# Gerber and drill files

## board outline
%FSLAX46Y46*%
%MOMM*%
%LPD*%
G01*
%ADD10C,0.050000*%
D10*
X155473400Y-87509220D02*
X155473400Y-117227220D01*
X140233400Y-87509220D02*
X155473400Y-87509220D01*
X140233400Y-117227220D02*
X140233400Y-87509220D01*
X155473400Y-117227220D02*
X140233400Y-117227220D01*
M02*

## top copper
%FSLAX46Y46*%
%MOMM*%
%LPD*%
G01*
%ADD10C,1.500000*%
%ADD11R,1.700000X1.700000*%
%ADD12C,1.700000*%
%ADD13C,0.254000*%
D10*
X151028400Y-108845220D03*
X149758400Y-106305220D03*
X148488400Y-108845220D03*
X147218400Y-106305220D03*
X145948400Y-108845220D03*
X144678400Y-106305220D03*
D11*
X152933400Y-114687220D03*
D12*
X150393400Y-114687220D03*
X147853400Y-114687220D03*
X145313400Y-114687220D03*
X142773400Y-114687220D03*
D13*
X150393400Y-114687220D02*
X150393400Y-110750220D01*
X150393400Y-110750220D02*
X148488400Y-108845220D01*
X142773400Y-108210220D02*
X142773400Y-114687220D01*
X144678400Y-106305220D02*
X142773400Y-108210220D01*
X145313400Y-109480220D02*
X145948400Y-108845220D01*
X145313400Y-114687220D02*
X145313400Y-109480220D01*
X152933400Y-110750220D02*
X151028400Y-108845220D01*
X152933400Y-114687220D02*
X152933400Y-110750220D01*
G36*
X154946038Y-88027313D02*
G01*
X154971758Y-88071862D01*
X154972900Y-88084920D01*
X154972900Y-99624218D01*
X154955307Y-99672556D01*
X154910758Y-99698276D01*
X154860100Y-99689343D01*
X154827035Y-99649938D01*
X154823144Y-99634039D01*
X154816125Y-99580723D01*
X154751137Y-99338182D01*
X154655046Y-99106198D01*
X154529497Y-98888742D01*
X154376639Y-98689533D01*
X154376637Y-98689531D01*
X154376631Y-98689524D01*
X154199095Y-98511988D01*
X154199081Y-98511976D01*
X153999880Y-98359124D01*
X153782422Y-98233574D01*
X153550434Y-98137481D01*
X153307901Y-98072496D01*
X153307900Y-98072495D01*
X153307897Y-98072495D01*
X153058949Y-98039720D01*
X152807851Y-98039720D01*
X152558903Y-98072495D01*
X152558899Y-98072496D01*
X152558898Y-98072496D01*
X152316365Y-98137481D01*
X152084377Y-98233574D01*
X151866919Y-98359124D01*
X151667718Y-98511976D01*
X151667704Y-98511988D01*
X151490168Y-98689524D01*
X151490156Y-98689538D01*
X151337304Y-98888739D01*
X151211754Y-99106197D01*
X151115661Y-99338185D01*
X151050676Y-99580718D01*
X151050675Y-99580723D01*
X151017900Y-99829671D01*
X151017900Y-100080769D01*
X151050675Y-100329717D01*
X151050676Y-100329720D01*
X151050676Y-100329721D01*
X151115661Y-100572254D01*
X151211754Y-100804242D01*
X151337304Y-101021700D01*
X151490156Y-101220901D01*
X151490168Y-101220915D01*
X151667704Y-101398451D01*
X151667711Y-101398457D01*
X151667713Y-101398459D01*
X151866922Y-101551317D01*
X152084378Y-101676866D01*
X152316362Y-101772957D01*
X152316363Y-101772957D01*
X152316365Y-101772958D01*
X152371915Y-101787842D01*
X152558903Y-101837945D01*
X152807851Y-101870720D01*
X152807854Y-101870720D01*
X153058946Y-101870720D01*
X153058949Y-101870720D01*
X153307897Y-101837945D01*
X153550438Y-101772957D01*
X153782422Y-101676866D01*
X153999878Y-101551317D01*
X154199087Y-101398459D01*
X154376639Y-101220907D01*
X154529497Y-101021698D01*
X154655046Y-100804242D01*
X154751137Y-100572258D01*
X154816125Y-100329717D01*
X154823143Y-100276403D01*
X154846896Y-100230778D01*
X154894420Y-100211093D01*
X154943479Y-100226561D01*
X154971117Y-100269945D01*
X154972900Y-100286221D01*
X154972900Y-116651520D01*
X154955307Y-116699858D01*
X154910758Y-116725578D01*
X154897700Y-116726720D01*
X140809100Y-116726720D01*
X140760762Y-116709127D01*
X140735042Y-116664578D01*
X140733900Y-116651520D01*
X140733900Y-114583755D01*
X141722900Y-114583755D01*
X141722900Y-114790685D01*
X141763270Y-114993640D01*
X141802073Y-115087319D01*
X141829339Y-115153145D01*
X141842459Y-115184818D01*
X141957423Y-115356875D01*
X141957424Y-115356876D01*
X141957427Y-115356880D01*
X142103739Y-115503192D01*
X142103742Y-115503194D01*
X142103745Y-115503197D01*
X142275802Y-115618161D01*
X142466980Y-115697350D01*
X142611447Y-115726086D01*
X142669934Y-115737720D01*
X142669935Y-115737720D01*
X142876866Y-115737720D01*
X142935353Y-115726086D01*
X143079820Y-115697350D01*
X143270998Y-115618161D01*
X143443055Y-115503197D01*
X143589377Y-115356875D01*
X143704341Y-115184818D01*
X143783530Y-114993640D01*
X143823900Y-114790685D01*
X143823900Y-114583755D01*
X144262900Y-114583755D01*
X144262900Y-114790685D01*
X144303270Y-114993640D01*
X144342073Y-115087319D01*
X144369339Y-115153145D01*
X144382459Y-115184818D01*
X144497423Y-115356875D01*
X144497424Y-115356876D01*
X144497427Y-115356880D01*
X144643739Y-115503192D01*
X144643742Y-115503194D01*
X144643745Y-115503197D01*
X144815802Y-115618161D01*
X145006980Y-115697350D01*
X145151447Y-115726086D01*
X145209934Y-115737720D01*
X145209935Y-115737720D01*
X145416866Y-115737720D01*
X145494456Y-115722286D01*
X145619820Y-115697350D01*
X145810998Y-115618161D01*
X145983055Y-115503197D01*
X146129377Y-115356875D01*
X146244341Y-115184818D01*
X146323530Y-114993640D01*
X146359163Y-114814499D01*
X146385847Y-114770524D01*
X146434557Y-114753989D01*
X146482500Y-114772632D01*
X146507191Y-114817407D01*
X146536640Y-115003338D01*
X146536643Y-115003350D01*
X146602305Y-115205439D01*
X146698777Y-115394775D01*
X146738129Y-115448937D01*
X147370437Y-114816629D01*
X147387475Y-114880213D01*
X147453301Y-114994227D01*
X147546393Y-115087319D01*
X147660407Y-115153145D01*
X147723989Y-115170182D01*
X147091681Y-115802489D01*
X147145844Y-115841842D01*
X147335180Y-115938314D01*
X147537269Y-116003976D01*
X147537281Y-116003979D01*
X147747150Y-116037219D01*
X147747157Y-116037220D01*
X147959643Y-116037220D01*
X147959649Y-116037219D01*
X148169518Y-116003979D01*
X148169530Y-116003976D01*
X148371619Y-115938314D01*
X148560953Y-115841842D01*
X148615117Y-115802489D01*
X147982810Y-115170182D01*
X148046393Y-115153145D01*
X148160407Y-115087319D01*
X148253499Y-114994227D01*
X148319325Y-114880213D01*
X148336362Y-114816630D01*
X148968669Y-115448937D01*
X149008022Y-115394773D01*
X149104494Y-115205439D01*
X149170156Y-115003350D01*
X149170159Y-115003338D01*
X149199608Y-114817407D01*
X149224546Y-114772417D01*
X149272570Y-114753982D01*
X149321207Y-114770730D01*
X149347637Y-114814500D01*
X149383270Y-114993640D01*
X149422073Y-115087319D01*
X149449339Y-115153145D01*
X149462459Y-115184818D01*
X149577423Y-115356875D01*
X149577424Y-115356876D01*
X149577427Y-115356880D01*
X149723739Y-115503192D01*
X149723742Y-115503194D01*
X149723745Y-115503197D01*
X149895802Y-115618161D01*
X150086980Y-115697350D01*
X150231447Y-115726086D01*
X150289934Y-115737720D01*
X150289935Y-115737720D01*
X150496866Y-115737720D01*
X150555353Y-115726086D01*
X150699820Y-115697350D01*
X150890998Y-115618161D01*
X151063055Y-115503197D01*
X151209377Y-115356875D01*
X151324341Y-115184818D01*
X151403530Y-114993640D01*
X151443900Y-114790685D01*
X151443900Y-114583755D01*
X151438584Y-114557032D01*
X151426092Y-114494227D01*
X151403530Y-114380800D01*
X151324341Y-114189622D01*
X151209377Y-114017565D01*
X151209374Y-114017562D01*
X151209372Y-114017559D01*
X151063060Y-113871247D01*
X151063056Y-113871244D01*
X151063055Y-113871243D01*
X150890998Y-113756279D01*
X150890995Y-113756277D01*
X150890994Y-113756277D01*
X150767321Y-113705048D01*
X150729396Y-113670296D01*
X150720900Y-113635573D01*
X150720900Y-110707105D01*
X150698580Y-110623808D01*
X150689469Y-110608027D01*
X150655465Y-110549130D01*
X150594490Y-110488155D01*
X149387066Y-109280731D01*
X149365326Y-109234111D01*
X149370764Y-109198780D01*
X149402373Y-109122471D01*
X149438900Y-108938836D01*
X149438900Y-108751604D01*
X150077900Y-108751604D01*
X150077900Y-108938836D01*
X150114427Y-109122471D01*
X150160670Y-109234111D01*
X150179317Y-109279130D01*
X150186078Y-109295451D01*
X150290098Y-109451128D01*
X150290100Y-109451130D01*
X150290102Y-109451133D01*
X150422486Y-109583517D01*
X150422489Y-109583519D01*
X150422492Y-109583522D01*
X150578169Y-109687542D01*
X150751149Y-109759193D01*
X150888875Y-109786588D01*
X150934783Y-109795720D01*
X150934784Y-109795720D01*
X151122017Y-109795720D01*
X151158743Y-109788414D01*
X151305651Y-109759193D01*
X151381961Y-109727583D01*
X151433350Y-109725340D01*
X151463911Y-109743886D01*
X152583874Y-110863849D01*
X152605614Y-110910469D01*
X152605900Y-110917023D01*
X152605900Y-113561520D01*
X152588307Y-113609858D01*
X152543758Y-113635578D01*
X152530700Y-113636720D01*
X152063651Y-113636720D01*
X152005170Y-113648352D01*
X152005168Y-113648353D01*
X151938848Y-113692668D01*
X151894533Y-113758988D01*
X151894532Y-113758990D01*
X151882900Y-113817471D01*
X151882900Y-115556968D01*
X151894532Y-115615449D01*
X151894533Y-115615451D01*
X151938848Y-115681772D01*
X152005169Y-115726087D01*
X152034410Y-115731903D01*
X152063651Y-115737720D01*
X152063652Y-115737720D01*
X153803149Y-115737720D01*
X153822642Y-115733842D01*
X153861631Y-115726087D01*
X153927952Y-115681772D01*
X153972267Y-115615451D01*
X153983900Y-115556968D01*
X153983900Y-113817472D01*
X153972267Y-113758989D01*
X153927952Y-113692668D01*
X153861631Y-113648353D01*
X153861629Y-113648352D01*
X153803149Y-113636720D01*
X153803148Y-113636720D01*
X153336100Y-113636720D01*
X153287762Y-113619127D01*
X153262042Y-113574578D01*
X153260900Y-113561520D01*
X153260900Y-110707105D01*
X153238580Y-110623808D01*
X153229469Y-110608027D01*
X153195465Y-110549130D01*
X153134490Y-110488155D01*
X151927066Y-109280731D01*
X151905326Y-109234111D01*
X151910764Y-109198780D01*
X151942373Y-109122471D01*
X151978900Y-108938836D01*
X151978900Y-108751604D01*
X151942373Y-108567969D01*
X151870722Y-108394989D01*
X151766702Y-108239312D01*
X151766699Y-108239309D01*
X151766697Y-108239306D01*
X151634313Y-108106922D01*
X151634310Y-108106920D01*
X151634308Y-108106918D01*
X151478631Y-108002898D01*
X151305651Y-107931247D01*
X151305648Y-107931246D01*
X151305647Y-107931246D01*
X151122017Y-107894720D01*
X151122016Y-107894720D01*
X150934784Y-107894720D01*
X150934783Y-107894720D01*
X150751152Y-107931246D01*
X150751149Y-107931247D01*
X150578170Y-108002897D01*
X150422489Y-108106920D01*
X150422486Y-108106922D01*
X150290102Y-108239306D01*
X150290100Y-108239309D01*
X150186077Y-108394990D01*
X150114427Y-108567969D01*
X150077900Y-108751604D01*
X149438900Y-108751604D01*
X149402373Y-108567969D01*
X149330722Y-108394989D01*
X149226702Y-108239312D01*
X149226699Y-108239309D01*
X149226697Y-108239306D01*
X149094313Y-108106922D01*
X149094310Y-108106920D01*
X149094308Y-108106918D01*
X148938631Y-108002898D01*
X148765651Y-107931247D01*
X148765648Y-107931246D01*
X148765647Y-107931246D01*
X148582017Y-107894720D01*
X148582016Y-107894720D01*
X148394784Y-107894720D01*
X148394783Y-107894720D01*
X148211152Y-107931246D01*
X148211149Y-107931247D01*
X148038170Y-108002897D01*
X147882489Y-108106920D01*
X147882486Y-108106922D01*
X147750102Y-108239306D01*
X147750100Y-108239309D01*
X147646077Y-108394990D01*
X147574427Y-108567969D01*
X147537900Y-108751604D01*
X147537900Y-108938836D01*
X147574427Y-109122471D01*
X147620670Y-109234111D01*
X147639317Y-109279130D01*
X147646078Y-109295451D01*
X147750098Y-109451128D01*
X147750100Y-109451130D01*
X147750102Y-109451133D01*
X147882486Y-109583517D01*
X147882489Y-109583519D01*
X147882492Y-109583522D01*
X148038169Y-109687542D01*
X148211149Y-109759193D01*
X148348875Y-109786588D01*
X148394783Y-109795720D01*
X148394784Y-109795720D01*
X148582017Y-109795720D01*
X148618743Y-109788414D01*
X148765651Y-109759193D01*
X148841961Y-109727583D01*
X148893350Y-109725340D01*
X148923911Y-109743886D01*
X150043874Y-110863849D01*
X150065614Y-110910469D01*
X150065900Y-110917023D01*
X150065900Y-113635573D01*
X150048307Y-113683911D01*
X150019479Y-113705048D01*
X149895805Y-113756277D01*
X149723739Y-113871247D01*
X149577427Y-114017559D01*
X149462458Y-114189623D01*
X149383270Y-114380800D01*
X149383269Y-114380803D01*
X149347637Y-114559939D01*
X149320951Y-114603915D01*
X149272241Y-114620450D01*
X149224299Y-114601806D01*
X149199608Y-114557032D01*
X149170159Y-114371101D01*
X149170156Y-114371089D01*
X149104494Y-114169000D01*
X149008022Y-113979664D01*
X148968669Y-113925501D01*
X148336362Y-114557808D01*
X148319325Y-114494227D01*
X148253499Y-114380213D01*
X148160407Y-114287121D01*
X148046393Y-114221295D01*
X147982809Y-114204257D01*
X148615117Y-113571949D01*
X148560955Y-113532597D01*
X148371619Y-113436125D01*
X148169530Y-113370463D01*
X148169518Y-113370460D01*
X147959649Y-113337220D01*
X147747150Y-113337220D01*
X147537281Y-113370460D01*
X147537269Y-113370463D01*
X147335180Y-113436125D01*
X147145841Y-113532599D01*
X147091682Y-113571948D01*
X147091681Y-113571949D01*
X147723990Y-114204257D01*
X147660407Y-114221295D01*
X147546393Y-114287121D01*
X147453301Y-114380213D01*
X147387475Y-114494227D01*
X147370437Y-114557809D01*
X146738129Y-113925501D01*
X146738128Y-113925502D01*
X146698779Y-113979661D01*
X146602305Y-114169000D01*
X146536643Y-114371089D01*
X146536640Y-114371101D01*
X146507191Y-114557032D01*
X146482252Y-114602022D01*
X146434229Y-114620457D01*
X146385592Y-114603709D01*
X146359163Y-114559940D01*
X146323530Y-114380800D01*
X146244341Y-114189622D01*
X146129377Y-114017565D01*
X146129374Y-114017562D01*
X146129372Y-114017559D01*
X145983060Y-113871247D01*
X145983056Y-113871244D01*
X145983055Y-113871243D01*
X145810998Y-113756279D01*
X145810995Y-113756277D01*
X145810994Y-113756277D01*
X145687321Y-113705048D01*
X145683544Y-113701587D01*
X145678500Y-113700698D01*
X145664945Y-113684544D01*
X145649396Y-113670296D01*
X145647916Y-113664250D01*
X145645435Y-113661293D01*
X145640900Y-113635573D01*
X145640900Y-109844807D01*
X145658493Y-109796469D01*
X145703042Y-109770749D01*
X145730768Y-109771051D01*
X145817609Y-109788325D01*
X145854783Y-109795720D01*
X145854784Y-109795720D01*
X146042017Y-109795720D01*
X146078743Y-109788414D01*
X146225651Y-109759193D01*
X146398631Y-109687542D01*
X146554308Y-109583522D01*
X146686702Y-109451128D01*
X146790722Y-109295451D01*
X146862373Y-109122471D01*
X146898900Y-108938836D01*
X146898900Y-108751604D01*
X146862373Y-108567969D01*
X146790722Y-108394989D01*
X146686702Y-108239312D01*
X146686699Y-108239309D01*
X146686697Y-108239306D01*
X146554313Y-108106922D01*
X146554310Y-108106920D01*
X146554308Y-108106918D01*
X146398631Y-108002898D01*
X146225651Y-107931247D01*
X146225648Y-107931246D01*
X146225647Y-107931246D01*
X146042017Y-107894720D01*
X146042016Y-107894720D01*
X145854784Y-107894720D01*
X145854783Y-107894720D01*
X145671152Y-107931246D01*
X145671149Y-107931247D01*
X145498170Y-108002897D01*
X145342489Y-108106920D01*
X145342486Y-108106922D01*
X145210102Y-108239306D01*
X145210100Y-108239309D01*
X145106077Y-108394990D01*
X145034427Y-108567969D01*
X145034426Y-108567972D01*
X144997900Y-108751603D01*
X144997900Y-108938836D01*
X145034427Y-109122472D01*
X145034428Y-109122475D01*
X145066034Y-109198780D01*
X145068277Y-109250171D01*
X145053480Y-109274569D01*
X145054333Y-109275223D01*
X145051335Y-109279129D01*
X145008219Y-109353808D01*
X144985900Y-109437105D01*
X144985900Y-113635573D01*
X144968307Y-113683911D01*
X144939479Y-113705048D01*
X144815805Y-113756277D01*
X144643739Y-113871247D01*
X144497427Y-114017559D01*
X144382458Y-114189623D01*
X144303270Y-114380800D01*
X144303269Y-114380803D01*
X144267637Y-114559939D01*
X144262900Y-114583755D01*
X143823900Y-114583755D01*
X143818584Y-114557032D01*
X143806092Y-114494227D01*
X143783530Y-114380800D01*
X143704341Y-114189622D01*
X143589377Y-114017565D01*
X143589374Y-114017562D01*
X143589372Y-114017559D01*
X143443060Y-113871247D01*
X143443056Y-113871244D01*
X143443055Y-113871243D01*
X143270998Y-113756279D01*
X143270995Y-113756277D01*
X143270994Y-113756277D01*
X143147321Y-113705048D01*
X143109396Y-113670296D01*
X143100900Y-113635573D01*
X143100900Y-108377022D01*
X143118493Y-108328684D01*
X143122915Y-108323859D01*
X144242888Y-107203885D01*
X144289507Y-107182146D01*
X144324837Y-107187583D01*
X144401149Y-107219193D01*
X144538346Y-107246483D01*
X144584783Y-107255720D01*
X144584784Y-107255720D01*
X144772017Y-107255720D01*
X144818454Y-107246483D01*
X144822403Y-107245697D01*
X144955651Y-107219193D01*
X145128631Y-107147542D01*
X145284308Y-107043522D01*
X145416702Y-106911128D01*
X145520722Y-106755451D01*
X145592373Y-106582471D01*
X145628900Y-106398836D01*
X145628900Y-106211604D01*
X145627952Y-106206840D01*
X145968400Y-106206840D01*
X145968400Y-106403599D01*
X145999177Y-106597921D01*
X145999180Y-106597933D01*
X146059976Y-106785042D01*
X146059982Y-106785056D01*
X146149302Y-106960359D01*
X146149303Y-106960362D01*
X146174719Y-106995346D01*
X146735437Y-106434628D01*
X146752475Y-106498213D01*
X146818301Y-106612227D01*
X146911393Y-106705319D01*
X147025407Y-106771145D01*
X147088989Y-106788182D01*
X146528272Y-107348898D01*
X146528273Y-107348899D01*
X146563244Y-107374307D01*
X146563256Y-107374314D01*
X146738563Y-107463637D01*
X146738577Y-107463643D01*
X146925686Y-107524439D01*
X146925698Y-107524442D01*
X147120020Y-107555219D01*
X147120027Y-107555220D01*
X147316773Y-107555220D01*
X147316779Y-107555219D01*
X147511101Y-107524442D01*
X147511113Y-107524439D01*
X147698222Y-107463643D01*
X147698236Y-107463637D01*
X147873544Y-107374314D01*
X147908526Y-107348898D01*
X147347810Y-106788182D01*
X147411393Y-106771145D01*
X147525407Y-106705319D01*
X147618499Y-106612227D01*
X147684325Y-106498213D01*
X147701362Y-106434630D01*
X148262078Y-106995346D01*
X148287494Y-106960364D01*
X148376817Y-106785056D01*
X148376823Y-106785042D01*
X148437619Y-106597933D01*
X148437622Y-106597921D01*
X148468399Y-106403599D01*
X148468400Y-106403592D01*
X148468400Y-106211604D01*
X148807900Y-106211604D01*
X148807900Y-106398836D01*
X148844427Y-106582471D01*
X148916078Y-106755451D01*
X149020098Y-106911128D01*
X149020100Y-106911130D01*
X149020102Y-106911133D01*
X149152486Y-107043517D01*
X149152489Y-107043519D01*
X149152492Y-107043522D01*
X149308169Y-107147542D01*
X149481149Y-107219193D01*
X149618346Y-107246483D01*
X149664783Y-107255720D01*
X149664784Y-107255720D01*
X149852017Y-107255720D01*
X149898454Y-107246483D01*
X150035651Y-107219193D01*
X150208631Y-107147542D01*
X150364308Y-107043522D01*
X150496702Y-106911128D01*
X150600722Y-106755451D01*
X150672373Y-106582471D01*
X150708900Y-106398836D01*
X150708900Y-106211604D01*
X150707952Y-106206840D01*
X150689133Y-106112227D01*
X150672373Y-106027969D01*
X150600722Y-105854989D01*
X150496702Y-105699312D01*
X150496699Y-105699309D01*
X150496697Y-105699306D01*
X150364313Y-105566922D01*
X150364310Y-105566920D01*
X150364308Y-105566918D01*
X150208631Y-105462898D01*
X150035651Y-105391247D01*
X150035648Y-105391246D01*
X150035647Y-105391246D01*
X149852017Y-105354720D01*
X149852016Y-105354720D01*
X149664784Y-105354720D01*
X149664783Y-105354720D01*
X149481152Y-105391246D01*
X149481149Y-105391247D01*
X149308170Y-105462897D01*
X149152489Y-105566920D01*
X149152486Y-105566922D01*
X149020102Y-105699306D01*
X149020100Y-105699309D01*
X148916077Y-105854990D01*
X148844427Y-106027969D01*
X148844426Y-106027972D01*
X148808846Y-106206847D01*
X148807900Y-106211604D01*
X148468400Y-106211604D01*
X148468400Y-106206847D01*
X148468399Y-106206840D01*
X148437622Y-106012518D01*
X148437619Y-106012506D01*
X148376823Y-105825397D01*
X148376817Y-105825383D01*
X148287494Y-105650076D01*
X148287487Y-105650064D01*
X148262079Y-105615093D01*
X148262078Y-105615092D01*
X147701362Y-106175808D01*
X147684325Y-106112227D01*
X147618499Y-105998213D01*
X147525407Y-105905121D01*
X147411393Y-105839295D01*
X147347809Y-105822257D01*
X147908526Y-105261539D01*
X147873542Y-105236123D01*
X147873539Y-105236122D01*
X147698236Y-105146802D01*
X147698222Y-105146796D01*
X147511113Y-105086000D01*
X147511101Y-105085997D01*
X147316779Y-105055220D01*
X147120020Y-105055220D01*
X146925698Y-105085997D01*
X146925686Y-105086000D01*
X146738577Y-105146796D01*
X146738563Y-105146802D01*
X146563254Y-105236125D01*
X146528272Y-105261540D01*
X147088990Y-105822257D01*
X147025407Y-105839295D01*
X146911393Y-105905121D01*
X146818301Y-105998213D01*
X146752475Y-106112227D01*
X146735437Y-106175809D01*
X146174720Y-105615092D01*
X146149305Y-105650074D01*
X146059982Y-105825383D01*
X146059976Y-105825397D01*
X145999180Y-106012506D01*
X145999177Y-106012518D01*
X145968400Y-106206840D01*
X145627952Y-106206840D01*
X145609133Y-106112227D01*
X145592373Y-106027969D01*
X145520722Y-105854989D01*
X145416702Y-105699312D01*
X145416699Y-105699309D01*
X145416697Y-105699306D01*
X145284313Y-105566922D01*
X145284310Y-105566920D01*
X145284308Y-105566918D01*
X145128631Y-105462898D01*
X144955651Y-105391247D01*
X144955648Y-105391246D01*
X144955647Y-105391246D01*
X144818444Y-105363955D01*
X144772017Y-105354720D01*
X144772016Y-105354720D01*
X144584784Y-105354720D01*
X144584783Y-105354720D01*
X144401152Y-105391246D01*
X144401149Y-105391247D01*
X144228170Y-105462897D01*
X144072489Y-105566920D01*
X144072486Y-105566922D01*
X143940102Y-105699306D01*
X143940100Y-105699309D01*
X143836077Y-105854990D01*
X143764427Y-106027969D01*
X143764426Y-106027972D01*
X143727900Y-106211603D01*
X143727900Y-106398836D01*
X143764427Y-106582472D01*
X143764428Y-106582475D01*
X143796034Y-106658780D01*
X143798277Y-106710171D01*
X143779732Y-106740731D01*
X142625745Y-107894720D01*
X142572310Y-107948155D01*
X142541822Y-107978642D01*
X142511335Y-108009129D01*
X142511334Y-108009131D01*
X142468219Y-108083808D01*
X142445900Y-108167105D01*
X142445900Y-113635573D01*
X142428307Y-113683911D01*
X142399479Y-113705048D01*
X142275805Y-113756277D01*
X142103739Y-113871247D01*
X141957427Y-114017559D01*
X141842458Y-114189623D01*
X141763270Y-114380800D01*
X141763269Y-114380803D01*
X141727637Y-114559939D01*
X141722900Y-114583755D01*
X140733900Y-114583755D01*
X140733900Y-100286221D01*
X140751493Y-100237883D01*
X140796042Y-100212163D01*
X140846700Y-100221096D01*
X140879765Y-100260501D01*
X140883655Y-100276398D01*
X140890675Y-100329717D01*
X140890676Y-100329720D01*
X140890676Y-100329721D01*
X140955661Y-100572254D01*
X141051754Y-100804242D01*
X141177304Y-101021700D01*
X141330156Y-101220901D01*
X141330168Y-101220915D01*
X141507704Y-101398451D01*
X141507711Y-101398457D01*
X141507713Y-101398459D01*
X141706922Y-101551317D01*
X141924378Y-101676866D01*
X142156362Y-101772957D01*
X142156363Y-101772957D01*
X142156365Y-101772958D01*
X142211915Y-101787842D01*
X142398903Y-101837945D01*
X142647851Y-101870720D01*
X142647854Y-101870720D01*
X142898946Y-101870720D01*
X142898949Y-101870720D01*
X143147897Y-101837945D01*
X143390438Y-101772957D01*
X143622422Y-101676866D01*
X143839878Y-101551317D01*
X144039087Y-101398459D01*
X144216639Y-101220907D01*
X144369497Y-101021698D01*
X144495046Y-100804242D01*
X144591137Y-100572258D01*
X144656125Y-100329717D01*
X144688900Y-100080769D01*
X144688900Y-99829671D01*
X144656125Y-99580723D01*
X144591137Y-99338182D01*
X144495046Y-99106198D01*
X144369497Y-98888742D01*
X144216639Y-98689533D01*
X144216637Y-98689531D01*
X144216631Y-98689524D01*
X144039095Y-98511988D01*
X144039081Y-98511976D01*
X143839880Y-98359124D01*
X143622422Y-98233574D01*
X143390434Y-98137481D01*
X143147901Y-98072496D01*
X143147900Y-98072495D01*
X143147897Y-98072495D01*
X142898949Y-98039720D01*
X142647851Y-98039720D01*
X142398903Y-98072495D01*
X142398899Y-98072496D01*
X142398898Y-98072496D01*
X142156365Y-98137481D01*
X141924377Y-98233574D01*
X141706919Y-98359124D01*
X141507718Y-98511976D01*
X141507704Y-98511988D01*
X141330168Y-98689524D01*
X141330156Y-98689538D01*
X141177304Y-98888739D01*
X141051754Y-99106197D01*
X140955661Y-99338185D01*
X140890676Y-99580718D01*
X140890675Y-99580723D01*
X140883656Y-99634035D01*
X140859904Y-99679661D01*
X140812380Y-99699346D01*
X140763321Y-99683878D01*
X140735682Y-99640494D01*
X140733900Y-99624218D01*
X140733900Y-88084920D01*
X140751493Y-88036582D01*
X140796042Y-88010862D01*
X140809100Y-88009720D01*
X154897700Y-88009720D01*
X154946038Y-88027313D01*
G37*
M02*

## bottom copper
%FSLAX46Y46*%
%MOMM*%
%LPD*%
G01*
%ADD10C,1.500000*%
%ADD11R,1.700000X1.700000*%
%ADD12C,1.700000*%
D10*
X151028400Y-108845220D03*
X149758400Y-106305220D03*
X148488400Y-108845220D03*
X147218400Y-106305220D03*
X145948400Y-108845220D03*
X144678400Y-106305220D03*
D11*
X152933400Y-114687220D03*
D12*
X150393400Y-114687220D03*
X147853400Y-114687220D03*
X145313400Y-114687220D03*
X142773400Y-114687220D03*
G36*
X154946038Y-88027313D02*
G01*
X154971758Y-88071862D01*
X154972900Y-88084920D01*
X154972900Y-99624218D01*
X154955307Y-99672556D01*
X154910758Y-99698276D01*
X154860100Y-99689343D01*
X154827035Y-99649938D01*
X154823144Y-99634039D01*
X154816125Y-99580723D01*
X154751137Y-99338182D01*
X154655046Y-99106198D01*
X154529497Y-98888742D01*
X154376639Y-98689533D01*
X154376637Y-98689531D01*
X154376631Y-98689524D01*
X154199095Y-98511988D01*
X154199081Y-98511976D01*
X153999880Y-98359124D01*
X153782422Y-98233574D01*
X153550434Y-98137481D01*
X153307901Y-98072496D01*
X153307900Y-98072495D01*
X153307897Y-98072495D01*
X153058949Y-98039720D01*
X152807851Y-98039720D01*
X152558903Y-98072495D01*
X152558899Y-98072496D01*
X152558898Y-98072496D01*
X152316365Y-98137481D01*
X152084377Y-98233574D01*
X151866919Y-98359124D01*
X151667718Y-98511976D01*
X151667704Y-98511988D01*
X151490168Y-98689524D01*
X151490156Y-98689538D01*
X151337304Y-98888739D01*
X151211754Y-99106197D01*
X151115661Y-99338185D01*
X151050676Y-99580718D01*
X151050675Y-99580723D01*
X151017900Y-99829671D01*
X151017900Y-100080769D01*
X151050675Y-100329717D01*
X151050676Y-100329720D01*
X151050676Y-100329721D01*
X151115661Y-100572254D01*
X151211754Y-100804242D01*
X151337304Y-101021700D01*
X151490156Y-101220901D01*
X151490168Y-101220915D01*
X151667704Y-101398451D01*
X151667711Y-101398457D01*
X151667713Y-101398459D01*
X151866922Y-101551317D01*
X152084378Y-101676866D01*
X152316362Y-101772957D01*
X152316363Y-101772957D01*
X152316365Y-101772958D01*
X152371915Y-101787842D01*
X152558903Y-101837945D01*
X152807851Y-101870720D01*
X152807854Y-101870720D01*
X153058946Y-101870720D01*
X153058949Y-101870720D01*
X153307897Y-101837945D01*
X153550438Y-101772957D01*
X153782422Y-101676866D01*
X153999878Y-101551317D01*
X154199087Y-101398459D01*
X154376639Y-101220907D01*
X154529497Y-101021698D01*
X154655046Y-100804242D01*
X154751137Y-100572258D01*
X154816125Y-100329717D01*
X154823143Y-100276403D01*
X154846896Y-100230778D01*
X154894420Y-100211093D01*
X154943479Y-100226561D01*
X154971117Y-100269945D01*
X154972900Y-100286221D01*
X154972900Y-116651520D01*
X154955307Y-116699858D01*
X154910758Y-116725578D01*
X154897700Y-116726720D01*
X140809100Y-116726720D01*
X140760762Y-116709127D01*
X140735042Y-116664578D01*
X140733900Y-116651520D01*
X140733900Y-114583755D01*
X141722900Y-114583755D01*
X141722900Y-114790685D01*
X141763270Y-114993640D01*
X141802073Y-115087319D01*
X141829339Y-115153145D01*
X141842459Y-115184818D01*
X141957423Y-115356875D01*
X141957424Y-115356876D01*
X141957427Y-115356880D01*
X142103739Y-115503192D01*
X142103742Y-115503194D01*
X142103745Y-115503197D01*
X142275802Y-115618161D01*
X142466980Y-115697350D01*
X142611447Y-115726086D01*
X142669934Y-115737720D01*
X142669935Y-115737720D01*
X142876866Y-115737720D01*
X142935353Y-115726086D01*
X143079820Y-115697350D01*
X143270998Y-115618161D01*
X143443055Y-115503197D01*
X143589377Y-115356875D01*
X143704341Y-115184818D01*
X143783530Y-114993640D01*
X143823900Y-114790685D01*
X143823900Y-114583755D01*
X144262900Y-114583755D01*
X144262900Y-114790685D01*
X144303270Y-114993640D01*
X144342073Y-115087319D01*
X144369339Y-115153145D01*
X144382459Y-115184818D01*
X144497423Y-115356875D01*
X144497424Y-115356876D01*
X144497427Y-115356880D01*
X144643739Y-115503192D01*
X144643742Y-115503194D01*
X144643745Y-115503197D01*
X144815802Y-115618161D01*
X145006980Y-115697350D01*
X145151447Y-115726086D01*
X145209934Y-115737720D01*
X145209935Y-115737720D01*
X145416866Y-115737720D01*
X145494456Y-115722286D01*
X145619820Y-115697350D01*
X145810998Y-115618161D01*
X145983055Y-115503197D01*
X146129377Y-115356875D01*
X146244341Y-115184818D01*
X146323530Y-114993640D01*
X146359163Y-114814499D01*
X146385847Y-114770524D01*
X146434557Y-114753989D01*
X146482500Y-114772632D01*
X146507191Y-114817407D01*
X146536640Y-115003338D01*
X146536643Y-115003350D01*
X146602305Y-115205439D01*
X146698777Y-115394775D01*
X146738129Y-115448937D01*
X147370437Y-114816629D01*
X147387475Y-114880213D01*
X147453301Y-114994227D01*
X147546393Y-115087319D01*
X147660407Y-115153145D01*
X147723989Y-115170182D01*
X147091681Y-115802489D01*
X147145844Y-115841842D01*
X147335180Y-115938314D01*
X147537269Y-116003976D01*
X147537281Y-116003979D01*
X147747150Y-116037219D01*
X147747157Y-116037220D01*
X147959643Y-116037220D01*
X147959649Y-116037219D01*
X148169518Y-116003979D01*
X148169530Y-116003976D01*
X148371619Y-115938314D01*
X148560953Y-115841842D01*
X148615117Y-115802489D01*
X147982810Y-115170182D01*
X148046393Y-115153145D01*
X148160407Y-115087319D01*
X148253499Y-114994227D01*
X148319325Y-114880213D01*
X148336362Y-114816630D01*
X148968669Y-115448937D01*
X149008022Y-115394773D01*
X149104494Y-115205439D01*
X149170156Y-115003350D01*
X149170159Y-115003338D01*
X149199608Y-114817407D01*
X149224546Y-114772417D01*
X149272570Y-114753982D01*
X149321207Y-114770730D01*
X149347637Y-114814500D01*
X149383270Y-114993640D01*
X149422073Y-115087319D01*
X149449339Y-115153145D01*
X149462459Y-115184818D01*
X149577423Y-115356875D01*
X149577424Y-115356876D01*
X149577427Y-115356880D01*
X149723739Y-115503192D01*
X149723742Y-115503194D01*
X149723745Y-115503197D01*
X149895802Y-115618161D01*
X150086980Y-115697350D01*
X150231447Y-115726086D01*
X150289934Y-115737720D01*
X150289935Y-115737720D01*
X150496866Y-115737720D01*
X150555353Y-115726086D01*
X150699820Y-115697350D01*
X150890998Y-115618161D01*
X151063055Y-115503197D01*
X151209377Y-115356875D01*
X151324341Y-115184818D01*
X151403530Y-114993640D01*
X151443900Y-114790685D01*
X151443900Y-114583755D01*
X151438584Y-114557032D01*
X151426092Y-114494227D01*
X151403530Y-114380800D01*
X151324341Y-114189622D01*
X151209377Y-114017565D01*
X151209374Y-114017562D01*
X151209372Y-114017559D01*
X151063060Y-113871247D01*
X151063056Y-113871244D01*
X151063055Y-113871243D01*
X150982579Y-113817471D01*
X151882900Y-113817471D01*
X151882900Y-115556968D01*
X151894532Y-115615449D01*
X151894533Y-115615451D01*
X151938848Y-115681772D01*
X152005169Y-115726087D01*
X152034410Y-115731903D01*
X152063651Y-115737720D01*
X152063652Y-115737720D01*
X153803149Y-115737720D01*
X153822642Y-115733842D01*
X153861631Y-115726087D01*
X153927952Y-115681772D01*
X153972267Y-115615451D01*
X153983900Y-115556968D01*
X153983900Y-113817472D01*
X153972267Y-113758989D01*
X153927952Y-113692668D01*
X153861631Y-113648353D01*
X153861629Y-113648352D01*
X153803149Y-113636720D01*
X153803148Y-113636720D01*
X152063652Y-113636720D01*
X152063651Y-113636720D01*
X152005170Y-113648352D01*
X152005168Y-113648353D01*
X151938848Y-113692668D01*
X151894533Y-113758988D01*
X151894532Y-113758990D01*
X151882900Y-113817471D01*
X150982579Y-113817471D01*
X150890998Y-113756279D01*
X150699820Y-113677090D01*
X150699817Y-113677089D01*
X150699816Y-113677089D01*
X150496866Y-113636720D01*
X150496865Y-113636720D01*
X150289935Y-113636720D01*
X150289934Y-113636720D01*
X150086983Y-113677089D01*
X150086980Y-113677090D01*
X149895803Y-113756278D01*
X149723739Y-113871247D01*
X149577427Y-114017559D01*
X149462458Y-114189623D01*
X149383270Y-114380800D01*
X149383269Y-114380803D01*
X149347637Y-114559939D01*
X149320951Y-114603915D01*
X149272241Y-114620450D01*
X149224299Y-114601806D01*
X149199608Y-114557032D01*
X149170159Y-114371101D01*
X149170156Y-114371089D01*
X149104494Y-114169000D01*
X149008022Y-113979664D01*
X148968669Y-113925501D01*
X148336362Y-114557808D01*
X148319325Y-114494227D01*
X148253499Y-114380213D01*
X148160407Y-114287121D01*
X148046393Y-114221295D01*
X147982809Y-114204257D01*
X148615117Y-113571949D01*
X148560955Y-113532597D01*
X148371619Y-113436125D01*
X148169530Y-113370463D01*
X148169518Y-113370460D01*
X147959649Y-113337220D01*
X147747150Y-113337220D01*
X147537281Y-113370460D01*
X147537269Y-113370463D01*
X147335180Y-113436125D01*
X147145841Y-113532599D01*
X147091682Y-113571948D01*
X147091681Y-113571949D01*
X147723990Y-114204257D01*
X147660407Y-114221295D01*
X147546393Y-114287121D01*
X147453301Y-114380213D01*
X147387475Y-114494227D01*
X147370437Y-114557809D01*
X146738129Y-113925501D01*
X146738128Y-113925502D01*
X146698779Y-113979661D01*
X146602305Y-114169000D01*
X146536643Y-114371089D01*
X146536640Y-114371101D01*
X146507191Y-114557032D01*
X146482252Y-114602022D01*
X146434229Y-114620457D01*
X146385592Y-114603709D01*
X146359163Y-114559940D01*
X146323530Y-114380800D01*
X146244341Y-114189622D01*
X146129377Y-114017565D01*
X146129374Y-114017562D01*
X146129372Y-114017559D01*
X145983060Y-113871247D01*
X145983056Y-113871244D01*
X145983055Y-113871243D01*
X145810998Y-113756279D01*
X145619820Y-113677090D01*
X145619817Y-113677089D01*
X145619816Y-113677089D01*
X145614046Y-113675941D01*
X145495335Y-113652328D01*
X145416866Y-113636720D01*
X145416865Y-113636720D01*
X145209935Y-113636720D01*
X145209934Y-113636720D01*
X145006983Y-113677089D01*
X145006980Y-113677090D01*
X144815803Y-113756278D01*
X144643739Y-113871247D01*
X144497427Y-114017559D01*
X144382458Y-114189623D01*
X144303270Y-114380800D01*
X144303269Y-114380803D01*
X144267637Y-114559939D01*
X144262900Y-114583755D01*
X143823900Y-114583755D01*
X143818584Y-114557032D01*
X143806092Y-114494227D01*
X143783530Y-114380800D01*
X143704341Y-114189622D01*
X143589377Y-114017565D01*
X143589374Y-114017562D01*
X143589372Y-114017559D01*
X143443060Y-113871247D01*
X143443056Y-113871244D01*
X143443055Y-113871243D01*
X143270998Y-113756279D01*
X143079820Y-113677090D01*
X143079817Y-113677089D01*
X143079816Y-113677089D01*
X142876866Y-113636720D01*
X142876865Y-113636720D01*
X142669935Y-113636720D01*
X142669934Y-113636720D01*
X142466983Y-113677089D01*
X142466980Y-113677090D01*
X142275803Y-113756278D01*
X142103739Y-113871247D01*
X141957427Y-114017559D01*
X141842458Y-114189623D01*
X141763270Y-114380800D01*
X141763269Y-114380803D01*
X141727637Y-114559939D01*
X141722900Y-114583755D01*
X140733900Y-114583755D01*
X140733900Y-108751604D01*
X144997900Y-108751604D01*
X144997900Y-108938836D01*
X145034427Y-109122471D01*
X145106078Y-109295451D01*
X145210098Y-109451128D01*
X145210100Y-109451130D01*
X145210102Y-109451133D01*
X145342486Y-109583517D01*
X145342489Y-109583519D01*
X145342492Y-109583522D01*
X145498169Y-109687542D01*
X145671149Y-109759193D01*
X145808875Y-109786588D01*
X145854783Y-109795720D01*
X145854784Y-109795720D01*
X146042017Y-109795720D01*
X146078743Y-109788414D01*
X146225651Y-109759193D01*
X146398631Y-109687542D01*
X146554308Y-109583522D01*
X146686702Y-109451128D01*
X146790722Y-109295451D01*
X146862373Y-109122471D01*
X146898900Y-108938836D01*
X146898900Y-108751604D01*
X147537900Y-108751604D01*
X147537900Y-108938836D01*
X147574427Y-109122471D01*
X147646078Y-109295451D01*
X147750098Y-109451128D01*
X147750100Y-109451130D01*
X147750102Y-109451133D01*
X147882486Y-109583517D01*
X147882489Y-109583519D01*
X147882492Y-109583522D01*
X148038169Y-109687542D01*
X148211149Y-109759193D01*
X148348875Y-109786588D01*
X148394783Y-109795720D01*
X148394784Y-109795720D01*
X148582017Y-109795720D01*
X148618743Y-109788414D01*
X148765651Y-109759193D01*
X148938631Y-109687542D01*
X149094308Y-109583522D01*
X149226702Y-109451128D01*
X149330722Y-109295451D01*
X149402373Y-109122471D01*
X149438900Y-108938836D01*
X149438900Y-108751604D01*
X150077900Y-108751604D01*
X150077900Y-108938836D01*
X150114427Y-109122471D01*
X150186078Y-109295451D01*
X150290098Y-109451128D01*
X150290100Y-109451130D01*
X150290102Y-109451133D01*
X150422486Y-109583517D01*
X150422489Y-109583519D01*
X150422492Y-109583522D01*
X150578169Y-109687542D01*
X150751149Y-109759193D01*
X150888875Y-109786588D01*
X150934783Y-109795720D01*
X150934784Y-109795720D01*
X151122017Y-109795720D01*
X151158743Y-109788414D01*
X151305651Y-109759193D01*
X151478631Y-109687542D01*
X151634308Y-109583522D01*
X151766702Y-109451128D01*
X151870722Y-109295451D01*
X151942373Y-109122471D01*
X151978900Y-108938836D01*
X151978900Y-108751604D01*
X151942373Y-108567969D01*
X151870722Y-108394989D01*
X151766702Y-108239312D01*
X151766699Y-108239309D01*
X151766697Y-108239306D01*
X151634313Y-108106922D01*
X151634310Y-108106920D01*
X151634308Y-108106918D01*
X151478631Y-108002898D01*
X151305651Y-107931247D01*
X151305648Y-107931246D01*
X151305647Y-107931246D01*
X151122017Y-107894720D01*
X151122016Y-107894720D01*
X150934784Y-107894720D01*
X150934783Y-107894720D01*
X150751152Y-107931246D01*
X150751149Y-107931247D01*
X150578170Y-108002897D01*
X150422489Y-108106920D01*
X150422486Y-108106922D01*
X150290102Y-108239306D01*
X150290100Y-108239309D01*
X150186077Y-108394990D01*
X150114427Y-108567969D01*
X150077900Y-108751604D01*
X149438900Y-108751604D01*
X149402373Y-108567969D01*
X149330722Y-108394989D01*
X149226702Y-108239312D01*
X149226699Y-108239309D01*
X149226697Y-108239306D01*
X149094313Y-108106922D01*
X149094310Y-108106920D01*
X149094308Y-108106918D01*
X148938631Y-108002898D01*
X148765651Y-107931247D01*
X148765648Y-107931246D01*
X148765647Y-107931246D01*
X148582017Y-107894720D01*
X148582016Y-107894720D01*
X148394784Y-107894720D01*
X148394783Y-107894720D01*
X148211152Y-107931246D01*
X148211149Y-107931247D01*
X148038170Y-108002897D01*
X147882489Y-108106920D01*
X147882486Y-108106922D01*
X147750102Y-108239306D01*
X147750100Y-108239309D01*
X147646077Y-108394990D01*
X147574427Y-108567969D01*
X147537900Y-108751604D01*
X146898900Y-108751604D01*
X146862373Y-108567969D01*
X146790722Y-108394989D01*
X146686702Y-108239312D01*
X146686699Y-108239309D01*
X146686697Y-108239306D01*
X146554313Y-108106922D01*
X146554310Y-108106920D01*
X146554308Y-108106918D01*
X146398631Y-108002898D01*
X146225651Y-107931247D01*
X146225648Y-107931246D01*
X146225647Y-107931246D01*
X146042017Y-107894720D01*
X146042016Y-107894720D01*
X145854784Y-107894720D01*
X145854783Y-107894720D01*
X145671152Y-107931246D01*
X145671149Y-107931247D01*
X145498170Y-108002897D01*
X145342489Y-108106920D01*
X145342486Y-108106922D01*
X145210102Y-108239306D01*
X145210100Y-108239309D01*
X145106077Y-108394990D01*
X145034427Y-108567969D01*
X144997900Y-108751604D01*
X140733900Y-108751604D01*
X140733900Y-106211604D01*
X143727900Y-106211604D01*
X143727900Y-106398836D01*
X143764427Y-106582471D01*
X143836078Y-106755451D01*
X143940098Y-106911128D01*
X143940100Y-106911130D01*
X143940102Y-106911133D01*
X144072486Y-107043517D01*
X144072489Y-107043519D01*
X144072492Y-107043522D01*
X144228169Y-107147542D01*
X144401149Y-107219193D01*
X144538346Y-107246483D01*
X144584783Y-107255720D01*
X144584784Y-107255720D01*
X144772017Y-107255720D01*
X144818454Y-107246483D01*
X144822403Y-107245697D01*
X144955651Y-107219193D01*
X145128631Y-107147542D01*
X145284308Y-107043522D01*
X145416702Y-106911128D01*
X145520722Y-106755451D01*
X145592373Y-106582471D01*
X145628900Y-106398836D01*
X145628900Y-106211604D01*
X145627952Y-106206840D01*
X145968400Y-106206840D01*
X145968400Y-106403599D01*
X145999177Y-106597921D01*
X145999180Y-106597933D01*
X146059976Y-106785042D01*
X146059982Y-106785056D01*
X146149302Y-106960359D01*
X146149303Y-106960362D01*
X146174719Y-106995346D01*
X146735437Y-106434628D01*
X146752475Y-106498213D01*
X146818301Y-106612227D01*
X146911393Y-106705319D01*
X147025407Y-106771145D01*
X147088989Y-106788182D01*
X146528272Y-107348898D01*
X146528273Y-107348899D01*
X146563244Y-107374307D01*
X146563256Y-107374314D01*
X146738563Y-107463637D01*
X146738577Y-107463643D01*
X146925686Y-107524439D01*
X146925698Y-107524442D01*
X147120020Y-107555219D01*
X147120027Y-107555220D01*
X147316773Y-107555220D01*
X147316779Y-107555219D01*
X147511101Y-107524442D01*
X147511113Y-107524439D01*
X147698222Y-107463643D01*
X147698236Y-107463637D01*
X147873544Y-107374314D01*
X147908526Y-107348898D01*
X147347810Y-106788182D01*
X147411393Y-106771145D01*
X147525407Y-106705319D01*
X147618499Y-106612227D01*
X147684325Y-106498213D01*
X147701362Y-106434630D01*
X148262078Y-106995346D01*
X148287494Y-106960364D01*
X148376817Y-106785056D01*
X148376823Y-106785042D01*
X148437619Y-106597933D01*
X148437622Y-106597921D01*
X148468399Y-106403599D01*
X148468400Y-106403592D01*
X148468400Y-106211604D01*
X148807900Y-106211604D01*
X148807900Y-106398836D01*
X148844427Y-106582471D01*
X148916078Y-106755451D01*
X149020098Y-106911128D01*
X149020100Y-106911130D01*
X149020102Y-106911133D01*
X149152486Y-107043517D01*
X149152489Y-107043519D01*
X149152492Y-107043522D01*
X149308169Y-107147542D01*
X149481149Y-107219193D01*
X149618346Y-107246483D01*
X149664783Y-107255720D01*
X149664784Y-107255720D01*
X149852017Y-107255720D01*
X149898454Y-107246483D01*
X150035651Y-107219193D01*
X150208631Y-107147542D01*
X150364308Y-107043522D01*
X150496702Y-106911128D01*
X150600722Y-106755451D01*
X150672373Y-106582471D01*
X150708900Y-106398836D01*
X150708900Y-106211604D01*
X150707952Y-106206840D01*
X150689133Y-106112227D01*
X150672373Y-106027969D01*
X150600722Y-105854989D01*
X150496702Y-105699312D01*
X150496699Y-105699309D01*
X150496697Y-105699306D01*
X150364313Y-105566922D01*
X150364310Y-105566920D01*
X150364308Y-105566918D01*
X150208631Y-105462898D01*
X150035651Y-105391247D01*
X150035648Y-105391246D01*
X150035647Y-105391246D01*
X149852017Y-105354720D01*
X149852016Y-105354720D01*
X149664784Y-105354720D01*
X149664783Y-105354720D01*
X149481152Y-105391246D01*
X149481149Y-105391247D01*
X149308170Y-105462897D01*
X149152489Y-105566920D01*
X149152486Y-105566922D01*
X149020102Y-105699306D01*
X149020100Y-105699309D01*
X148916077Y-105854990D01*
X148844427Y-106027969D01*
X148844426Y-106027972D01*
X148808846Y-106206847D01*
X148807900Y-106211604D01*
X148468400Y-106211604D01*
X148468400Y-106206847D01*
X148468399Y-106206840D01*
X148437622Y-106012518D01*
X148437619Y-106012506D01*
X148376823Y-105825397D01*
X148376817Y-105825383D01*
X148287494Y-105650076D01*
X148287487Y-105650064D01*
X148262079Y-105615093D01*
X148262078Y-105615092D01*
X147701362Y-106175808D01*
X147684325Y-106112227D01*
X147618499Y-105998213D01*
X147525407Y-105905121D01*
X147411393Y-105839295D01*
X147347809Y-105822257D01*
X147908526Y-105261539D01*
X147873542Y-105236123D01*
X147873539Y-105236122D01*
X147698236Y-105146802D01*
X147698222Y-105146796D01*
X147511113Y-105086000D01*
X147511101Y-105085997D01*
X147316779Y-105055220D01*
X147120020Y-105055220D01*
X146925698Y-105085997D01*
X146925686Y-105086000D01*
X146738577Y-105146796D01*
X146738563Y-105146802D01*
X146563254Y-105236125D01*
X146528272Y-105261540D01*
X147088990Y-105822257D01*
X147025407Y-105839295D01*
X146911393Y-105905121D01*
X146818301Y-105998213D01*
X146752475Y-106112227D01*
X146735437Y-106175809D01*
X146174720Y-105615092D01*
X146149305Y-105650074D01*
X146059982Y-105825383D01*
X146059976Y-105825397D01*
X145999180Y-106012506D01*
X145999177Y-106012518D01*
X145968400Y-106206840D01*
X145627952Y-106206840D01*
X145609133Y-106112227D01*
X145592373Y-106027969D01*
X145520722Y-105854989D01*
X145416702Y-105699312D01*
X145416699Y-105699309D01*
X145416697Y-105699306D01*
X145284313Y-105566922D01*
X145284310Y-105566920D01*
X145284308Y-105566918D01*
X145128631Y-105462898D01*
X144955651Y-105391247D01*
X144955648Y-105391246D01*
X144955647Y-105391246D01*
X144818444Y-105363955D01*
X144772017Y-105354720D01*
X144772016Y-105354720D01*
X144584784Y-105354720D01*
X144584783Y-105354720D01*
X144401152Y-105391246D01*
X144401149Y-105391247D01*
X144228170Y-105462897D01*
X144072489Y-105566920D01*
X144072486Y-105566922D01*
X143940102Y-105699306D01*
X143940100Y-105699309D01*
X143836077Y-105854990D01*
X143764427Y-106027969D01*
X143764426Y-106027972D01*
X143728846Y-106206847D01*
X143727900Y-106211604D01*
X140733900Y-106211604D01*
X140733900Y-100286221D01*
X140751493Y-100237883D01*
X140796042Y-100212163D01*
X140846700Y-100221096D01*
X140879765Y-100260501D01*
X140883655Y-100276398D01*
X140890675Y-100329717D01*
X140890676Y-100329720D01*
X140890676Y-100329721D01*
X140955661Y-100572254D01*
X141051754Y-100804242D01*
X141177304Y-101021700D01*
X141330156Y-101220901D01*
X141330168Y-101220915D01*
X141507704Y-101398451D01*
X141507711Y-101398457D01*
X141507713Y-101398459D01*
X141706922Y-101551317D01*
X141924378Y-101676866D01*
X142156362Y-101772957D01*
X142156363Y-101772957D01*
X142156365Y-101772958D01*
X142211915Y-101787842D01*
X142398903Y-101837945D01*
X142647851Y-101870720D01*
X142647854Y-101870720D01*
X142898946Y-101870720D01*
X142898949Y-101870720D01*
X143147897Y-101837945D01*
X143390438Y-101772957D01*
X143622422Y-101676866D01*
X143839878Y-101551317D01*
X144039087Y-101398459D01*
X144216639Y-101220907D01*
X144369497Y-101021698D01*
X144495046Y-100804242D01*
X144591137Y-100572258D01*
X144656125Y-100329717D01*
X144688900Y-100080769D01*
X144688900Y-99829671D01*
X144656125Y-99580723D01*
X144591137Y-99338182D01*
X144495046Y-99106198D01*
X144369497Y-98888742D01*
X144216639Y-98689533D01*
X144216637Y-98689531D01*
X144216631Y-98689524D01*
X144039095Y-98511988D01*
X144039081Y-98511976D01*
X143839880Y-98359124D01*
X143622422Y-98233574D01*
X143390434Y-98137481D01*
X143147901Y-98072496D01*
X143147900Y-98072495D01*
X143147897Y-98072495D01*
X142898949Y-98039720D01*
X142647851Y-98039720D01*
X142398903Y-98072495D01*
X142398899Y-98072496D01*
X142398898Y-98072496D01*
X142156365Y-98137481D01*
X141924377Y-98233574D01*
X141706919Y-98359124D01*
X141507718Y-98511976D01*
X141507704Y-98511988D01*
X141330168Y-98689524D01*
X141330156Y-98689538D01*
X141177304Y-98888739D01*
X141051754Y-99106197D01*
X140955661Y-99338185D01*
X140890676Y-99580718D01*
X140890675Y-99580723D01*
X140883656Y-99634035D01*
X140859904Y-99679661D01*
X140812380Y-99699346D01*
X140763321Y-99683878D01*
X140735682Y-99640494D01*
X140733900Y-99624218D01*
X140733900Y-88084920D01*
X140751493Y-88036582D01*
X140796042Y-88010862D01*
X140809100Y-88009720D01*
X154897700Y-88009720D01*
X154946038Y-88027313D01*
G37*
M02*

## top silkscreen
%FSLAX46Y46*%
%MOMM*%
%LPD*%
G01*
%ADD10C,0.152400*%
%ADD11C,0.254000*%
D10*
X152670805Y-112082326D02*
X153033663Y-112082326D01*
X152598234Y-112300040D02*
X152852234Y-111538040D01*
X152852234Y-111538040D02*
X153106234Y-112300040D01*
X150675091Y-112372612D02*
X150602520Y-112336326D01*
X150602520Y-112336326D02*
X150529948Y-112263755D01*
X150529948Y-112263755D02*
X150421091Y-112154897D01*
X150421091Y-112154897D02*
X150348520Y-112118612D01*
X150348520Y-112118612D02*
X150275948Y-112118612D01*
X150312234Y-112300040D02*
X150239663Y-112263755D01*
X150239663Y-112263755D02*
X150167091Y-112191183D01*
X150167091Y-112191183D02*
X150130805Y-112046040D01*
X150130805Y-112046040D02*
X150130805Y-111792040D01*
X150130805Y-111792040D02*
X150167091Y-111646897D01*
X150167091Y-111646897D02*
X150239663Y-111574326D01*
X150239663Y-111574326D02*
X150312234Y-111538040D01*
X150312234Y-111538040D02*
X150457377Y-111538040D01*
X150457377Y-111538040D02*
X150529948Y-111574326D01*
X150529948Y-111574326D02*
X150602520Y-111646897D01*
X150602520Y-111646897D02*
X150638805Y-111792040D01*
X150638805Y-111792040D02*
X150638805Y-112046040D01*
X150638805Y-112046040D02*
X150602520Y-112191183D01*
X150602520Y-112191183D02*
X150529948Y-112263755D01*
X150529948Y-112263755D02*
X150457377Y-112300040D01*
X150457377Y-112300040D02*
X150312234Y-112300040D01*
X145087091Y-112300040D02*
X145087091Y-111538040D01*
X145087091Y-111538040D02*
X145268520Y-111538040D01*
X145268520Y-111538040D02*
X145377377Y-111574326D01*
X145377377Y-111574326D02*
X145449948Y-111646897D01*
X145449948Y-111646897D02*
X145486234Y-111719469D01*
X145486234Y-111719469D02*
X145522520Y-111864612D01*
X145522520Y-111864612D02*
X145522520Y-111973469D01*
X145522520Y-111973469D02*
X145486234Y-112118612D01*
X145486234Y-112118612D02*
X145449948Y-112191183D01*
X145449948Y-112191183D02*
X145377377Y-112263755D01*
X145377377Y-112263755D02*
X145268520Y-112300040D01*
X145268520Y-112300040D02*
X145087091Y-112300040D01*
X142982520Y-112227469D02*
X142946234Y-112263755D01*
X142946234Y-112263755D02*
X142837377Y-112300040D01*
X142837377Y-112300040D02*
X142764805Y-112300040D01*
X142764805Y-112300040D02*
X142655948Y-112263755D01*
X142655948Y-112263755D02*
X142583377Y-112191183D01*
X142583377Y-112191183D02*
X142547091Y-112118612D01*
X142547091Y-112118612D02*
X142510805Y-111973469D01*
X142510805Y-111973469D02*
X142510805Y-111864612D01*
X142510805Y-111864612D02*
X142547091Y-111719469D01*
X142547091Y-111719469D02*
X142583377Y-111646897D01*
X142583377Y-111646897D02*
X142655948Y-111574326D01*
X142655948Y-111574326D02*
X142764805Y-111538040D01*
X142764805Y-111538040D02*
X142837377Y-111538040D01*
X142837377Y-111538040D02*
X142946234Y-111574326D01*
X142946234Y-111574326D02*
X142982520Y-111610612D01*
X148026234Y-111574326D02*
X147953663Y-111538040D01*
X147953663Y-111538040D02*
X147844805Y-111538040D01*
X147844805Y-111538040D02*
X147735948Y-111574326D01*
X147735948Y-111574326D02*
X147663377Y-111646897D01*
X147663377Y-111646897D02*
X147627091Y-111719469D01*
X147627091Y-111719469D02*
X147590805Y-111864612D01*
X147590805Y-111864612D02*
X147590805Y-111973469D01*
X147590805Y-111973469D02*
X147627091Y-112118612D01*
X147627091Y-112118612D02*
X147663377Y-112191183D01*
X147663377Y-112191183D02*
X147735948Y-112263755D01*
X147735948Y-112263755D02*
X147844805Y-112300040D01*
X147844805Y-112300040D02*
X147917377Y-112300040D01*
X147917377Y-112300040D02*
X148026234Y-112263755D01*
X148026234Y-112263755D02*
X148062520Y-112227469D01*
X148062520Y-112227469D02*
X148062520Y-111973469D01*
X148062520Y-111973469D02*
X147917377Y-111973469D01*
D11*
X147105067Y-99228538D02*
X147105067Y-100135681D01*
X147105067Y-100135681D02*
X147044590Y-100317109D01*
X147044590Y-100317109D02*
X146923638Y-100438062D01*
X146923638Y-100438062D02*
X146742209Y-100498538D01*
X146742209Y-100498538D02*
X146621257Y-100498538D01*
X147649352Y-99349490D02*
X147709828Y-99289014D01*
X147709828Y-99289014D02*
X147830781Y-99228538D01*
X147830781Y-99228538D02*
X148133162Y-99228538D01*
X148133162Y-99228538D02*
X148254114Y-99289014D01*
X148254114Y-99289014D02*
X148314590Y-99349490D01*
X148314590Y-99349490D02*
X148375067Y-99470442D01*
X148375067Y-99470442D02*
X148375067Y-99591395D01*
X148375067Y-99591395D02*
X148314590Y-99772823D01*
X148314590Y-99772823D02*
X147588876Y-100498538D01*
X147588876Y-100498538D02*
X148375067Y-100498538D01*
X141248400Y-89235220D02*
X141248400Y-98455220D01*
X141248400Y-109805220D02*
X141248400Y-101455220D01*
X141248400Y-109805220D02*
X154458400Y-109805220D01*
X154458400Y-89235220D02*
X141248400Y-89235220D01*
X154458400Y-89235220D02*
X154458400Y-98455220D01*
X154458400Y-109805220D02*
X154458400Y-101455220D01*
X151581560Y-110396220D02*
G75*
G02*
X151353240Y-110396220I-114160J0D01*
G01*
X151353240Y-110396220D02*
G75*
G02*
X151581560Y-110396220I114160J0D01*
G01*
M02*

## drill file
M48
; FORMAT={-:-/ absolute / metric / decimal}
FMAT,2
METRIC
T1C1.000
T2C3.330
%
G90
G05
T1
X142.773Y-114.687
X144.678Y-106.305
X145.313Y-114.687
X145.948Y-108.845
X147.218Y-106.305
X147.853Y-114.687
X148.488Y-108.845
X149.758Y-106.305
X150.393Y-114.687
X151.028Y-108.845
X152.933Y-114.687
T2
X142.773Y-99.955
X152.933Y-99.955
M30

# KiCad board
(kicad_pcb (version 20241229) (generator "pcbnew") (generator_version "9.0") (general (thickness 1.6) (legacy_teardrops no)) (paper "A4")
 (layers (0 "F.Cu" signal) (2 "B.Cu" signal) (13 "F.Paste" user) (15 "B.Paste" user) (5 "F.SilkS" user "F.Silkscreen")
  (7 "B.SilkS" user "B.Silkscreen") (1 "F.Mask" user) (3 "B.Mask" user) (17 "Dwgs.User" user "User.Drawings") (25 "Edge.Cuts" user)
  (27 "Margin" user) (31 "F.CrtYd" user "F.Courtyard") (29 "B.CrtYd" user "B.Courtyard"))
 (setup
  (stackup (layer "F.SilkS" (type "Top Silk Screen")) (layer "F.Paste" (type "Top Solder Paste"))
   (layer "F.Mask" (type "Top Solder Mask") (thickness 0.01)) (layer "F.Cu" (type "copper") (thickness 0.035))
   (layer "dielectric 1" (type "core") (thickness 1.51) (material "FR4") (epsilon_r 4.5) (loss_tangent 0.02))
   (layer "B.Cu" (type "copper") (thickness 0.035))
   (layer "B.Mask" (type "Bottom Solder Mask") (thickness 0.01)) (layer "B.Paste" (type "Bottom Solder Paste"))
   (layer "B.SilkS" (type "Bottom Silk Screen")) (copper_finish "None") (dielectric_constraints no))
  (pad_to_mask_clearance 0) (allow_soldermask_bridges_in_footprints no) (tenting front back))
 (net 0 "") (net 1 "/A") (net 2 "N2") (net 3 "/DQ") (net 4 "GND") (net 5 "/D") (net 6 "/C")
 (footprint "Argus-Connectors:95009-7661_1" (layer "F.Cu") (at 147.8534 99.95522)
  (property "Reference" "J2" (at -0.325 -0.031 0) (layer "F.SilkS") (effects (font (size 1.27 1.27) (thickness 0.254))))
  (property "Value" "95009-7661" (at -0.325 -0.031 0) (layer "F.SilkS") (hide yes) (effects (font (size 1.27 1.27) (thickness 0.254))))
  (fp_line (start -6.605 -10.72) (end -6.605 -1.5) (stroke (width 0.254) (type solid)) (layer "F.SilkS"))
  (fp_line (start -6.605 9.85) (end -6.605 1.5) (stroke (width 0.254) (type solid)) (layer "F.SilkS"))
  (fp_line (start -6.605 9.85) (end 6.605 9.85) (stroke (width 0.254) (type solid)) (layer "F.SilkS"))
  (fp_line (start 6.605 -10.72) (end -6.605 -10.72) (stroke (width 0.254) (type solid)) (layer "F.SilkS"))
  (fp_line (start 6.605 -10.72) (end 6.605 -1.5) (stroke (width 0.254) (type solid)) (layer "F.SilkS"))
  (fp_line (start 6.605 9.85) (end 6.605 1.5) (stroke (width 0.254) (type solid)) (layer "F.SilkS"))
  (fp_circle (center 3.614 10.441) (end 3.614 10.55516) (stroke (width 0.254) (type solid)) (fill no) (layer "F.SilkS"))
  (pad "" np_thru_hole circle (at -5.08 0) (size 3.33 3.33) (drill 3.33) (layers "*.Cu" "*.Mask"))
  (pad "" np_thru_hole circle (at 5.08 0) (size 3.33 3.33) (drill 3.33) (layers "*.Cu" "*.Mask"))
  (pad "1" thru_hole circle (at 3.175 8.89) (size 1.5 1.5) (drill 1) (layers "*.Cu" "*.Mask") (remove_unused_layers no) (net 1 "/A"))
  (pad "2" thru_hole circle (at 1.905 6.35) (size 1.5 1.5) (drill 1) (layers "*.Cu" "*.Mask") (remove_unused_layers no) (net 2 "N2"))
  (pad "3" thru_hole circle (at 0.635 8.89) (size 1.5 1.5) (drill 1) (layers "*.Cu" "*.Mask") (remove_unused_layers no) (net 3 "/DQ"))
  (pad "4" thru_hole circle (at -0.635 6.35) (size 1.5 1.5) (drill 1) (layers "*.Cu" "*.Mask") (remove_unused_layers no) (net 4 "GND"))
  (pad "5" thru_hole circle (at -1.905 8.89) (size 1.5 1.5) (drill 1) (layers "*.Cu" "*.Mask") (remove_unused_layers no) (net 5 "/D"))
  (pad "6" thru_hole circle (at -3.175 6.35) (size 1.5 1.5) (drill 1) (layers "*.Cu" "*.Mask") (remove_unused_layers no) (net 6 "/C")))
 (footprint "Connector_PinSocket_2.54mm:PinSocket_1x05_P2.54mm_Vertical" (layer "B.Cu") (at 152.9334 114.68722 90)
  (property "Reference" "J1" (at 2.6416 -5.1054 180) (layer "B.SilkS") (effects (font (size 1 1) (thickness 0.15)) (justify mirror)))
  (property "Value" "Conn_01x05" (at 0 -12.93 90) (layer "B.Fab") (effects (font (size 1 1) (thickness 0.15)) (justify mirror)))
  (pad "1" thru_hole rect (at 0 0 90) (size 1.7 1.7) (drill 1) (layers "*.Cu" "*.Mask") (remove_unused_layers no) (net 1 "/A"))
  (pad "2" thru_hole circle (at 0 -2.54 90) (size 1.7 1.7) (drill 1) (layers "*.Cu" "*.Mask") (remove_unused_layers no) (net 3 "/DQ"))
  (pad "3" thru_hole circle (at 0 -5.08 90) (size 1.7 1.7) (drill 1) (layers "*.Cu" "*.Mask") (remove_unused_layers no) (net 4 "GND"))
  (pad "4" thru_hole circle (at 0 -7.62 90) (size 1.7 1.7) (drill 1) (layers "*.Cu" "*.Mask") (remove_unused_layers no) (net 5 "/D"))
  (pad "5" thru_hole circle (at 0 -10.16 90) (size 1.7 1.7) (drill 1) (layers "*.Cu" "*.Mask") (remove_unused_layers no) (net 6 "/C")))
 (gr_line (start 155.4734 87.50922) (end 155.4734 117.22722) (stroke (width 0.05) (type default)) (layer "Edge.Cuts"))
 (gr_line (start 140.2334 87.50922) (end 155.4734 87.50922) (stroke (width 0.05) (type default)) (layer "Edge.Cuts"))
 (gr_line (start 140.2334 117.22722) (end 140.2334 87.50922) (stroke (width 0.05) (type default)) (layer "Edge.Cuts"))
 (gr_line (start 155.4734 117.22722) (end 140.2334 117.22722) (stroke (width 0.05) (type default)) (layer "Edge.Cuts"))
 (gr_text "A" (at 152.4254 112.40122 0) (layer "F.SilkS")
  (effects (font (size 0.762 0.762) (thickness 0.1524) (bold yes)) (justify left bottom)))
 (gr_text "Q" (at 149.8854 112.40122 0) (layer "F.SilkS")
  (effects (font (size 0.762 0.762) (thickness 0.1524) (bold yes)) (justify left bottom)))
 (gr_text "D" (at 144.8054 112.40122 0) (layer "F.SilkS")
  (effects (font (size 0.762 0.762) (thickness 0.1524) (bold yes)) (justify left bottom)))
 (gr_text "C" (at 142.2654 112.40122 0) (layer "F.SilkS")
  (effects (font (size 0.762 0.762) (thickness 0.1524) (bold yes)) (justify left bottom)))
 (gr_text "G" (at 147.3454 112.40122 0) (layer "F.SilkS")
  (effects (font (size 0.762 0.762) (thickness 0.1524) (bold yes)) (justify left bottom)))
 (segment (start 150.3934 114.68722) (end 150.3934 110.75022) (width 0.254) (layer "F.Cu") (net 3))
 (segment (start 150.3934 110.75022) (end 148.4884 108.84522) (width 0.254) (layer "F.Cu") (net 3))
 (segment (start 142.7734 108.21022) (end 142.7734 114.68722) (width 0.254) (layer "F.Cu") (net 6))
 (segment (start 144.6784 106.30522) (end 142.7734 108.21022) (width 0.254) (layer "F.Cu") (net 6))
 (segment (start 145.3134 109.48022) (end 145.9484 108.84522) (width 0.254) (layer "F.Cu") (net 5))
 (segment (start 145.3134 114.68722) (end 145.3134 109.48022) (width 0.254) (layer "F.Cu") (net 5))
 (segment (start 152.9334 110.75022) (end 151.0284 108.84522) (width 0.254) (layer "F.Cu") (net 1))
 (segment (start 152.9334 114.68722) (end 152.9334 110.75022) (width 0.254) (layer "F.Cu") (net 1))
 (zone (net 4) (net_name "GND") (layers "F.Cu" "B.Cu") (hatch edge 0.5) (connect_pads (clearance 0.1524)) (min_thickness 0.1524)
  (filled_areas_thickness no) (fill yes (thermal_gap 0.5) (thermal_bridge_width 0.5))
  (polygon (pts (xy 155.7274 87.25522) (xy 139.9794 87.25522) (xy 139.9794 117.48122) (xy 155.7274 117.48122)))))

